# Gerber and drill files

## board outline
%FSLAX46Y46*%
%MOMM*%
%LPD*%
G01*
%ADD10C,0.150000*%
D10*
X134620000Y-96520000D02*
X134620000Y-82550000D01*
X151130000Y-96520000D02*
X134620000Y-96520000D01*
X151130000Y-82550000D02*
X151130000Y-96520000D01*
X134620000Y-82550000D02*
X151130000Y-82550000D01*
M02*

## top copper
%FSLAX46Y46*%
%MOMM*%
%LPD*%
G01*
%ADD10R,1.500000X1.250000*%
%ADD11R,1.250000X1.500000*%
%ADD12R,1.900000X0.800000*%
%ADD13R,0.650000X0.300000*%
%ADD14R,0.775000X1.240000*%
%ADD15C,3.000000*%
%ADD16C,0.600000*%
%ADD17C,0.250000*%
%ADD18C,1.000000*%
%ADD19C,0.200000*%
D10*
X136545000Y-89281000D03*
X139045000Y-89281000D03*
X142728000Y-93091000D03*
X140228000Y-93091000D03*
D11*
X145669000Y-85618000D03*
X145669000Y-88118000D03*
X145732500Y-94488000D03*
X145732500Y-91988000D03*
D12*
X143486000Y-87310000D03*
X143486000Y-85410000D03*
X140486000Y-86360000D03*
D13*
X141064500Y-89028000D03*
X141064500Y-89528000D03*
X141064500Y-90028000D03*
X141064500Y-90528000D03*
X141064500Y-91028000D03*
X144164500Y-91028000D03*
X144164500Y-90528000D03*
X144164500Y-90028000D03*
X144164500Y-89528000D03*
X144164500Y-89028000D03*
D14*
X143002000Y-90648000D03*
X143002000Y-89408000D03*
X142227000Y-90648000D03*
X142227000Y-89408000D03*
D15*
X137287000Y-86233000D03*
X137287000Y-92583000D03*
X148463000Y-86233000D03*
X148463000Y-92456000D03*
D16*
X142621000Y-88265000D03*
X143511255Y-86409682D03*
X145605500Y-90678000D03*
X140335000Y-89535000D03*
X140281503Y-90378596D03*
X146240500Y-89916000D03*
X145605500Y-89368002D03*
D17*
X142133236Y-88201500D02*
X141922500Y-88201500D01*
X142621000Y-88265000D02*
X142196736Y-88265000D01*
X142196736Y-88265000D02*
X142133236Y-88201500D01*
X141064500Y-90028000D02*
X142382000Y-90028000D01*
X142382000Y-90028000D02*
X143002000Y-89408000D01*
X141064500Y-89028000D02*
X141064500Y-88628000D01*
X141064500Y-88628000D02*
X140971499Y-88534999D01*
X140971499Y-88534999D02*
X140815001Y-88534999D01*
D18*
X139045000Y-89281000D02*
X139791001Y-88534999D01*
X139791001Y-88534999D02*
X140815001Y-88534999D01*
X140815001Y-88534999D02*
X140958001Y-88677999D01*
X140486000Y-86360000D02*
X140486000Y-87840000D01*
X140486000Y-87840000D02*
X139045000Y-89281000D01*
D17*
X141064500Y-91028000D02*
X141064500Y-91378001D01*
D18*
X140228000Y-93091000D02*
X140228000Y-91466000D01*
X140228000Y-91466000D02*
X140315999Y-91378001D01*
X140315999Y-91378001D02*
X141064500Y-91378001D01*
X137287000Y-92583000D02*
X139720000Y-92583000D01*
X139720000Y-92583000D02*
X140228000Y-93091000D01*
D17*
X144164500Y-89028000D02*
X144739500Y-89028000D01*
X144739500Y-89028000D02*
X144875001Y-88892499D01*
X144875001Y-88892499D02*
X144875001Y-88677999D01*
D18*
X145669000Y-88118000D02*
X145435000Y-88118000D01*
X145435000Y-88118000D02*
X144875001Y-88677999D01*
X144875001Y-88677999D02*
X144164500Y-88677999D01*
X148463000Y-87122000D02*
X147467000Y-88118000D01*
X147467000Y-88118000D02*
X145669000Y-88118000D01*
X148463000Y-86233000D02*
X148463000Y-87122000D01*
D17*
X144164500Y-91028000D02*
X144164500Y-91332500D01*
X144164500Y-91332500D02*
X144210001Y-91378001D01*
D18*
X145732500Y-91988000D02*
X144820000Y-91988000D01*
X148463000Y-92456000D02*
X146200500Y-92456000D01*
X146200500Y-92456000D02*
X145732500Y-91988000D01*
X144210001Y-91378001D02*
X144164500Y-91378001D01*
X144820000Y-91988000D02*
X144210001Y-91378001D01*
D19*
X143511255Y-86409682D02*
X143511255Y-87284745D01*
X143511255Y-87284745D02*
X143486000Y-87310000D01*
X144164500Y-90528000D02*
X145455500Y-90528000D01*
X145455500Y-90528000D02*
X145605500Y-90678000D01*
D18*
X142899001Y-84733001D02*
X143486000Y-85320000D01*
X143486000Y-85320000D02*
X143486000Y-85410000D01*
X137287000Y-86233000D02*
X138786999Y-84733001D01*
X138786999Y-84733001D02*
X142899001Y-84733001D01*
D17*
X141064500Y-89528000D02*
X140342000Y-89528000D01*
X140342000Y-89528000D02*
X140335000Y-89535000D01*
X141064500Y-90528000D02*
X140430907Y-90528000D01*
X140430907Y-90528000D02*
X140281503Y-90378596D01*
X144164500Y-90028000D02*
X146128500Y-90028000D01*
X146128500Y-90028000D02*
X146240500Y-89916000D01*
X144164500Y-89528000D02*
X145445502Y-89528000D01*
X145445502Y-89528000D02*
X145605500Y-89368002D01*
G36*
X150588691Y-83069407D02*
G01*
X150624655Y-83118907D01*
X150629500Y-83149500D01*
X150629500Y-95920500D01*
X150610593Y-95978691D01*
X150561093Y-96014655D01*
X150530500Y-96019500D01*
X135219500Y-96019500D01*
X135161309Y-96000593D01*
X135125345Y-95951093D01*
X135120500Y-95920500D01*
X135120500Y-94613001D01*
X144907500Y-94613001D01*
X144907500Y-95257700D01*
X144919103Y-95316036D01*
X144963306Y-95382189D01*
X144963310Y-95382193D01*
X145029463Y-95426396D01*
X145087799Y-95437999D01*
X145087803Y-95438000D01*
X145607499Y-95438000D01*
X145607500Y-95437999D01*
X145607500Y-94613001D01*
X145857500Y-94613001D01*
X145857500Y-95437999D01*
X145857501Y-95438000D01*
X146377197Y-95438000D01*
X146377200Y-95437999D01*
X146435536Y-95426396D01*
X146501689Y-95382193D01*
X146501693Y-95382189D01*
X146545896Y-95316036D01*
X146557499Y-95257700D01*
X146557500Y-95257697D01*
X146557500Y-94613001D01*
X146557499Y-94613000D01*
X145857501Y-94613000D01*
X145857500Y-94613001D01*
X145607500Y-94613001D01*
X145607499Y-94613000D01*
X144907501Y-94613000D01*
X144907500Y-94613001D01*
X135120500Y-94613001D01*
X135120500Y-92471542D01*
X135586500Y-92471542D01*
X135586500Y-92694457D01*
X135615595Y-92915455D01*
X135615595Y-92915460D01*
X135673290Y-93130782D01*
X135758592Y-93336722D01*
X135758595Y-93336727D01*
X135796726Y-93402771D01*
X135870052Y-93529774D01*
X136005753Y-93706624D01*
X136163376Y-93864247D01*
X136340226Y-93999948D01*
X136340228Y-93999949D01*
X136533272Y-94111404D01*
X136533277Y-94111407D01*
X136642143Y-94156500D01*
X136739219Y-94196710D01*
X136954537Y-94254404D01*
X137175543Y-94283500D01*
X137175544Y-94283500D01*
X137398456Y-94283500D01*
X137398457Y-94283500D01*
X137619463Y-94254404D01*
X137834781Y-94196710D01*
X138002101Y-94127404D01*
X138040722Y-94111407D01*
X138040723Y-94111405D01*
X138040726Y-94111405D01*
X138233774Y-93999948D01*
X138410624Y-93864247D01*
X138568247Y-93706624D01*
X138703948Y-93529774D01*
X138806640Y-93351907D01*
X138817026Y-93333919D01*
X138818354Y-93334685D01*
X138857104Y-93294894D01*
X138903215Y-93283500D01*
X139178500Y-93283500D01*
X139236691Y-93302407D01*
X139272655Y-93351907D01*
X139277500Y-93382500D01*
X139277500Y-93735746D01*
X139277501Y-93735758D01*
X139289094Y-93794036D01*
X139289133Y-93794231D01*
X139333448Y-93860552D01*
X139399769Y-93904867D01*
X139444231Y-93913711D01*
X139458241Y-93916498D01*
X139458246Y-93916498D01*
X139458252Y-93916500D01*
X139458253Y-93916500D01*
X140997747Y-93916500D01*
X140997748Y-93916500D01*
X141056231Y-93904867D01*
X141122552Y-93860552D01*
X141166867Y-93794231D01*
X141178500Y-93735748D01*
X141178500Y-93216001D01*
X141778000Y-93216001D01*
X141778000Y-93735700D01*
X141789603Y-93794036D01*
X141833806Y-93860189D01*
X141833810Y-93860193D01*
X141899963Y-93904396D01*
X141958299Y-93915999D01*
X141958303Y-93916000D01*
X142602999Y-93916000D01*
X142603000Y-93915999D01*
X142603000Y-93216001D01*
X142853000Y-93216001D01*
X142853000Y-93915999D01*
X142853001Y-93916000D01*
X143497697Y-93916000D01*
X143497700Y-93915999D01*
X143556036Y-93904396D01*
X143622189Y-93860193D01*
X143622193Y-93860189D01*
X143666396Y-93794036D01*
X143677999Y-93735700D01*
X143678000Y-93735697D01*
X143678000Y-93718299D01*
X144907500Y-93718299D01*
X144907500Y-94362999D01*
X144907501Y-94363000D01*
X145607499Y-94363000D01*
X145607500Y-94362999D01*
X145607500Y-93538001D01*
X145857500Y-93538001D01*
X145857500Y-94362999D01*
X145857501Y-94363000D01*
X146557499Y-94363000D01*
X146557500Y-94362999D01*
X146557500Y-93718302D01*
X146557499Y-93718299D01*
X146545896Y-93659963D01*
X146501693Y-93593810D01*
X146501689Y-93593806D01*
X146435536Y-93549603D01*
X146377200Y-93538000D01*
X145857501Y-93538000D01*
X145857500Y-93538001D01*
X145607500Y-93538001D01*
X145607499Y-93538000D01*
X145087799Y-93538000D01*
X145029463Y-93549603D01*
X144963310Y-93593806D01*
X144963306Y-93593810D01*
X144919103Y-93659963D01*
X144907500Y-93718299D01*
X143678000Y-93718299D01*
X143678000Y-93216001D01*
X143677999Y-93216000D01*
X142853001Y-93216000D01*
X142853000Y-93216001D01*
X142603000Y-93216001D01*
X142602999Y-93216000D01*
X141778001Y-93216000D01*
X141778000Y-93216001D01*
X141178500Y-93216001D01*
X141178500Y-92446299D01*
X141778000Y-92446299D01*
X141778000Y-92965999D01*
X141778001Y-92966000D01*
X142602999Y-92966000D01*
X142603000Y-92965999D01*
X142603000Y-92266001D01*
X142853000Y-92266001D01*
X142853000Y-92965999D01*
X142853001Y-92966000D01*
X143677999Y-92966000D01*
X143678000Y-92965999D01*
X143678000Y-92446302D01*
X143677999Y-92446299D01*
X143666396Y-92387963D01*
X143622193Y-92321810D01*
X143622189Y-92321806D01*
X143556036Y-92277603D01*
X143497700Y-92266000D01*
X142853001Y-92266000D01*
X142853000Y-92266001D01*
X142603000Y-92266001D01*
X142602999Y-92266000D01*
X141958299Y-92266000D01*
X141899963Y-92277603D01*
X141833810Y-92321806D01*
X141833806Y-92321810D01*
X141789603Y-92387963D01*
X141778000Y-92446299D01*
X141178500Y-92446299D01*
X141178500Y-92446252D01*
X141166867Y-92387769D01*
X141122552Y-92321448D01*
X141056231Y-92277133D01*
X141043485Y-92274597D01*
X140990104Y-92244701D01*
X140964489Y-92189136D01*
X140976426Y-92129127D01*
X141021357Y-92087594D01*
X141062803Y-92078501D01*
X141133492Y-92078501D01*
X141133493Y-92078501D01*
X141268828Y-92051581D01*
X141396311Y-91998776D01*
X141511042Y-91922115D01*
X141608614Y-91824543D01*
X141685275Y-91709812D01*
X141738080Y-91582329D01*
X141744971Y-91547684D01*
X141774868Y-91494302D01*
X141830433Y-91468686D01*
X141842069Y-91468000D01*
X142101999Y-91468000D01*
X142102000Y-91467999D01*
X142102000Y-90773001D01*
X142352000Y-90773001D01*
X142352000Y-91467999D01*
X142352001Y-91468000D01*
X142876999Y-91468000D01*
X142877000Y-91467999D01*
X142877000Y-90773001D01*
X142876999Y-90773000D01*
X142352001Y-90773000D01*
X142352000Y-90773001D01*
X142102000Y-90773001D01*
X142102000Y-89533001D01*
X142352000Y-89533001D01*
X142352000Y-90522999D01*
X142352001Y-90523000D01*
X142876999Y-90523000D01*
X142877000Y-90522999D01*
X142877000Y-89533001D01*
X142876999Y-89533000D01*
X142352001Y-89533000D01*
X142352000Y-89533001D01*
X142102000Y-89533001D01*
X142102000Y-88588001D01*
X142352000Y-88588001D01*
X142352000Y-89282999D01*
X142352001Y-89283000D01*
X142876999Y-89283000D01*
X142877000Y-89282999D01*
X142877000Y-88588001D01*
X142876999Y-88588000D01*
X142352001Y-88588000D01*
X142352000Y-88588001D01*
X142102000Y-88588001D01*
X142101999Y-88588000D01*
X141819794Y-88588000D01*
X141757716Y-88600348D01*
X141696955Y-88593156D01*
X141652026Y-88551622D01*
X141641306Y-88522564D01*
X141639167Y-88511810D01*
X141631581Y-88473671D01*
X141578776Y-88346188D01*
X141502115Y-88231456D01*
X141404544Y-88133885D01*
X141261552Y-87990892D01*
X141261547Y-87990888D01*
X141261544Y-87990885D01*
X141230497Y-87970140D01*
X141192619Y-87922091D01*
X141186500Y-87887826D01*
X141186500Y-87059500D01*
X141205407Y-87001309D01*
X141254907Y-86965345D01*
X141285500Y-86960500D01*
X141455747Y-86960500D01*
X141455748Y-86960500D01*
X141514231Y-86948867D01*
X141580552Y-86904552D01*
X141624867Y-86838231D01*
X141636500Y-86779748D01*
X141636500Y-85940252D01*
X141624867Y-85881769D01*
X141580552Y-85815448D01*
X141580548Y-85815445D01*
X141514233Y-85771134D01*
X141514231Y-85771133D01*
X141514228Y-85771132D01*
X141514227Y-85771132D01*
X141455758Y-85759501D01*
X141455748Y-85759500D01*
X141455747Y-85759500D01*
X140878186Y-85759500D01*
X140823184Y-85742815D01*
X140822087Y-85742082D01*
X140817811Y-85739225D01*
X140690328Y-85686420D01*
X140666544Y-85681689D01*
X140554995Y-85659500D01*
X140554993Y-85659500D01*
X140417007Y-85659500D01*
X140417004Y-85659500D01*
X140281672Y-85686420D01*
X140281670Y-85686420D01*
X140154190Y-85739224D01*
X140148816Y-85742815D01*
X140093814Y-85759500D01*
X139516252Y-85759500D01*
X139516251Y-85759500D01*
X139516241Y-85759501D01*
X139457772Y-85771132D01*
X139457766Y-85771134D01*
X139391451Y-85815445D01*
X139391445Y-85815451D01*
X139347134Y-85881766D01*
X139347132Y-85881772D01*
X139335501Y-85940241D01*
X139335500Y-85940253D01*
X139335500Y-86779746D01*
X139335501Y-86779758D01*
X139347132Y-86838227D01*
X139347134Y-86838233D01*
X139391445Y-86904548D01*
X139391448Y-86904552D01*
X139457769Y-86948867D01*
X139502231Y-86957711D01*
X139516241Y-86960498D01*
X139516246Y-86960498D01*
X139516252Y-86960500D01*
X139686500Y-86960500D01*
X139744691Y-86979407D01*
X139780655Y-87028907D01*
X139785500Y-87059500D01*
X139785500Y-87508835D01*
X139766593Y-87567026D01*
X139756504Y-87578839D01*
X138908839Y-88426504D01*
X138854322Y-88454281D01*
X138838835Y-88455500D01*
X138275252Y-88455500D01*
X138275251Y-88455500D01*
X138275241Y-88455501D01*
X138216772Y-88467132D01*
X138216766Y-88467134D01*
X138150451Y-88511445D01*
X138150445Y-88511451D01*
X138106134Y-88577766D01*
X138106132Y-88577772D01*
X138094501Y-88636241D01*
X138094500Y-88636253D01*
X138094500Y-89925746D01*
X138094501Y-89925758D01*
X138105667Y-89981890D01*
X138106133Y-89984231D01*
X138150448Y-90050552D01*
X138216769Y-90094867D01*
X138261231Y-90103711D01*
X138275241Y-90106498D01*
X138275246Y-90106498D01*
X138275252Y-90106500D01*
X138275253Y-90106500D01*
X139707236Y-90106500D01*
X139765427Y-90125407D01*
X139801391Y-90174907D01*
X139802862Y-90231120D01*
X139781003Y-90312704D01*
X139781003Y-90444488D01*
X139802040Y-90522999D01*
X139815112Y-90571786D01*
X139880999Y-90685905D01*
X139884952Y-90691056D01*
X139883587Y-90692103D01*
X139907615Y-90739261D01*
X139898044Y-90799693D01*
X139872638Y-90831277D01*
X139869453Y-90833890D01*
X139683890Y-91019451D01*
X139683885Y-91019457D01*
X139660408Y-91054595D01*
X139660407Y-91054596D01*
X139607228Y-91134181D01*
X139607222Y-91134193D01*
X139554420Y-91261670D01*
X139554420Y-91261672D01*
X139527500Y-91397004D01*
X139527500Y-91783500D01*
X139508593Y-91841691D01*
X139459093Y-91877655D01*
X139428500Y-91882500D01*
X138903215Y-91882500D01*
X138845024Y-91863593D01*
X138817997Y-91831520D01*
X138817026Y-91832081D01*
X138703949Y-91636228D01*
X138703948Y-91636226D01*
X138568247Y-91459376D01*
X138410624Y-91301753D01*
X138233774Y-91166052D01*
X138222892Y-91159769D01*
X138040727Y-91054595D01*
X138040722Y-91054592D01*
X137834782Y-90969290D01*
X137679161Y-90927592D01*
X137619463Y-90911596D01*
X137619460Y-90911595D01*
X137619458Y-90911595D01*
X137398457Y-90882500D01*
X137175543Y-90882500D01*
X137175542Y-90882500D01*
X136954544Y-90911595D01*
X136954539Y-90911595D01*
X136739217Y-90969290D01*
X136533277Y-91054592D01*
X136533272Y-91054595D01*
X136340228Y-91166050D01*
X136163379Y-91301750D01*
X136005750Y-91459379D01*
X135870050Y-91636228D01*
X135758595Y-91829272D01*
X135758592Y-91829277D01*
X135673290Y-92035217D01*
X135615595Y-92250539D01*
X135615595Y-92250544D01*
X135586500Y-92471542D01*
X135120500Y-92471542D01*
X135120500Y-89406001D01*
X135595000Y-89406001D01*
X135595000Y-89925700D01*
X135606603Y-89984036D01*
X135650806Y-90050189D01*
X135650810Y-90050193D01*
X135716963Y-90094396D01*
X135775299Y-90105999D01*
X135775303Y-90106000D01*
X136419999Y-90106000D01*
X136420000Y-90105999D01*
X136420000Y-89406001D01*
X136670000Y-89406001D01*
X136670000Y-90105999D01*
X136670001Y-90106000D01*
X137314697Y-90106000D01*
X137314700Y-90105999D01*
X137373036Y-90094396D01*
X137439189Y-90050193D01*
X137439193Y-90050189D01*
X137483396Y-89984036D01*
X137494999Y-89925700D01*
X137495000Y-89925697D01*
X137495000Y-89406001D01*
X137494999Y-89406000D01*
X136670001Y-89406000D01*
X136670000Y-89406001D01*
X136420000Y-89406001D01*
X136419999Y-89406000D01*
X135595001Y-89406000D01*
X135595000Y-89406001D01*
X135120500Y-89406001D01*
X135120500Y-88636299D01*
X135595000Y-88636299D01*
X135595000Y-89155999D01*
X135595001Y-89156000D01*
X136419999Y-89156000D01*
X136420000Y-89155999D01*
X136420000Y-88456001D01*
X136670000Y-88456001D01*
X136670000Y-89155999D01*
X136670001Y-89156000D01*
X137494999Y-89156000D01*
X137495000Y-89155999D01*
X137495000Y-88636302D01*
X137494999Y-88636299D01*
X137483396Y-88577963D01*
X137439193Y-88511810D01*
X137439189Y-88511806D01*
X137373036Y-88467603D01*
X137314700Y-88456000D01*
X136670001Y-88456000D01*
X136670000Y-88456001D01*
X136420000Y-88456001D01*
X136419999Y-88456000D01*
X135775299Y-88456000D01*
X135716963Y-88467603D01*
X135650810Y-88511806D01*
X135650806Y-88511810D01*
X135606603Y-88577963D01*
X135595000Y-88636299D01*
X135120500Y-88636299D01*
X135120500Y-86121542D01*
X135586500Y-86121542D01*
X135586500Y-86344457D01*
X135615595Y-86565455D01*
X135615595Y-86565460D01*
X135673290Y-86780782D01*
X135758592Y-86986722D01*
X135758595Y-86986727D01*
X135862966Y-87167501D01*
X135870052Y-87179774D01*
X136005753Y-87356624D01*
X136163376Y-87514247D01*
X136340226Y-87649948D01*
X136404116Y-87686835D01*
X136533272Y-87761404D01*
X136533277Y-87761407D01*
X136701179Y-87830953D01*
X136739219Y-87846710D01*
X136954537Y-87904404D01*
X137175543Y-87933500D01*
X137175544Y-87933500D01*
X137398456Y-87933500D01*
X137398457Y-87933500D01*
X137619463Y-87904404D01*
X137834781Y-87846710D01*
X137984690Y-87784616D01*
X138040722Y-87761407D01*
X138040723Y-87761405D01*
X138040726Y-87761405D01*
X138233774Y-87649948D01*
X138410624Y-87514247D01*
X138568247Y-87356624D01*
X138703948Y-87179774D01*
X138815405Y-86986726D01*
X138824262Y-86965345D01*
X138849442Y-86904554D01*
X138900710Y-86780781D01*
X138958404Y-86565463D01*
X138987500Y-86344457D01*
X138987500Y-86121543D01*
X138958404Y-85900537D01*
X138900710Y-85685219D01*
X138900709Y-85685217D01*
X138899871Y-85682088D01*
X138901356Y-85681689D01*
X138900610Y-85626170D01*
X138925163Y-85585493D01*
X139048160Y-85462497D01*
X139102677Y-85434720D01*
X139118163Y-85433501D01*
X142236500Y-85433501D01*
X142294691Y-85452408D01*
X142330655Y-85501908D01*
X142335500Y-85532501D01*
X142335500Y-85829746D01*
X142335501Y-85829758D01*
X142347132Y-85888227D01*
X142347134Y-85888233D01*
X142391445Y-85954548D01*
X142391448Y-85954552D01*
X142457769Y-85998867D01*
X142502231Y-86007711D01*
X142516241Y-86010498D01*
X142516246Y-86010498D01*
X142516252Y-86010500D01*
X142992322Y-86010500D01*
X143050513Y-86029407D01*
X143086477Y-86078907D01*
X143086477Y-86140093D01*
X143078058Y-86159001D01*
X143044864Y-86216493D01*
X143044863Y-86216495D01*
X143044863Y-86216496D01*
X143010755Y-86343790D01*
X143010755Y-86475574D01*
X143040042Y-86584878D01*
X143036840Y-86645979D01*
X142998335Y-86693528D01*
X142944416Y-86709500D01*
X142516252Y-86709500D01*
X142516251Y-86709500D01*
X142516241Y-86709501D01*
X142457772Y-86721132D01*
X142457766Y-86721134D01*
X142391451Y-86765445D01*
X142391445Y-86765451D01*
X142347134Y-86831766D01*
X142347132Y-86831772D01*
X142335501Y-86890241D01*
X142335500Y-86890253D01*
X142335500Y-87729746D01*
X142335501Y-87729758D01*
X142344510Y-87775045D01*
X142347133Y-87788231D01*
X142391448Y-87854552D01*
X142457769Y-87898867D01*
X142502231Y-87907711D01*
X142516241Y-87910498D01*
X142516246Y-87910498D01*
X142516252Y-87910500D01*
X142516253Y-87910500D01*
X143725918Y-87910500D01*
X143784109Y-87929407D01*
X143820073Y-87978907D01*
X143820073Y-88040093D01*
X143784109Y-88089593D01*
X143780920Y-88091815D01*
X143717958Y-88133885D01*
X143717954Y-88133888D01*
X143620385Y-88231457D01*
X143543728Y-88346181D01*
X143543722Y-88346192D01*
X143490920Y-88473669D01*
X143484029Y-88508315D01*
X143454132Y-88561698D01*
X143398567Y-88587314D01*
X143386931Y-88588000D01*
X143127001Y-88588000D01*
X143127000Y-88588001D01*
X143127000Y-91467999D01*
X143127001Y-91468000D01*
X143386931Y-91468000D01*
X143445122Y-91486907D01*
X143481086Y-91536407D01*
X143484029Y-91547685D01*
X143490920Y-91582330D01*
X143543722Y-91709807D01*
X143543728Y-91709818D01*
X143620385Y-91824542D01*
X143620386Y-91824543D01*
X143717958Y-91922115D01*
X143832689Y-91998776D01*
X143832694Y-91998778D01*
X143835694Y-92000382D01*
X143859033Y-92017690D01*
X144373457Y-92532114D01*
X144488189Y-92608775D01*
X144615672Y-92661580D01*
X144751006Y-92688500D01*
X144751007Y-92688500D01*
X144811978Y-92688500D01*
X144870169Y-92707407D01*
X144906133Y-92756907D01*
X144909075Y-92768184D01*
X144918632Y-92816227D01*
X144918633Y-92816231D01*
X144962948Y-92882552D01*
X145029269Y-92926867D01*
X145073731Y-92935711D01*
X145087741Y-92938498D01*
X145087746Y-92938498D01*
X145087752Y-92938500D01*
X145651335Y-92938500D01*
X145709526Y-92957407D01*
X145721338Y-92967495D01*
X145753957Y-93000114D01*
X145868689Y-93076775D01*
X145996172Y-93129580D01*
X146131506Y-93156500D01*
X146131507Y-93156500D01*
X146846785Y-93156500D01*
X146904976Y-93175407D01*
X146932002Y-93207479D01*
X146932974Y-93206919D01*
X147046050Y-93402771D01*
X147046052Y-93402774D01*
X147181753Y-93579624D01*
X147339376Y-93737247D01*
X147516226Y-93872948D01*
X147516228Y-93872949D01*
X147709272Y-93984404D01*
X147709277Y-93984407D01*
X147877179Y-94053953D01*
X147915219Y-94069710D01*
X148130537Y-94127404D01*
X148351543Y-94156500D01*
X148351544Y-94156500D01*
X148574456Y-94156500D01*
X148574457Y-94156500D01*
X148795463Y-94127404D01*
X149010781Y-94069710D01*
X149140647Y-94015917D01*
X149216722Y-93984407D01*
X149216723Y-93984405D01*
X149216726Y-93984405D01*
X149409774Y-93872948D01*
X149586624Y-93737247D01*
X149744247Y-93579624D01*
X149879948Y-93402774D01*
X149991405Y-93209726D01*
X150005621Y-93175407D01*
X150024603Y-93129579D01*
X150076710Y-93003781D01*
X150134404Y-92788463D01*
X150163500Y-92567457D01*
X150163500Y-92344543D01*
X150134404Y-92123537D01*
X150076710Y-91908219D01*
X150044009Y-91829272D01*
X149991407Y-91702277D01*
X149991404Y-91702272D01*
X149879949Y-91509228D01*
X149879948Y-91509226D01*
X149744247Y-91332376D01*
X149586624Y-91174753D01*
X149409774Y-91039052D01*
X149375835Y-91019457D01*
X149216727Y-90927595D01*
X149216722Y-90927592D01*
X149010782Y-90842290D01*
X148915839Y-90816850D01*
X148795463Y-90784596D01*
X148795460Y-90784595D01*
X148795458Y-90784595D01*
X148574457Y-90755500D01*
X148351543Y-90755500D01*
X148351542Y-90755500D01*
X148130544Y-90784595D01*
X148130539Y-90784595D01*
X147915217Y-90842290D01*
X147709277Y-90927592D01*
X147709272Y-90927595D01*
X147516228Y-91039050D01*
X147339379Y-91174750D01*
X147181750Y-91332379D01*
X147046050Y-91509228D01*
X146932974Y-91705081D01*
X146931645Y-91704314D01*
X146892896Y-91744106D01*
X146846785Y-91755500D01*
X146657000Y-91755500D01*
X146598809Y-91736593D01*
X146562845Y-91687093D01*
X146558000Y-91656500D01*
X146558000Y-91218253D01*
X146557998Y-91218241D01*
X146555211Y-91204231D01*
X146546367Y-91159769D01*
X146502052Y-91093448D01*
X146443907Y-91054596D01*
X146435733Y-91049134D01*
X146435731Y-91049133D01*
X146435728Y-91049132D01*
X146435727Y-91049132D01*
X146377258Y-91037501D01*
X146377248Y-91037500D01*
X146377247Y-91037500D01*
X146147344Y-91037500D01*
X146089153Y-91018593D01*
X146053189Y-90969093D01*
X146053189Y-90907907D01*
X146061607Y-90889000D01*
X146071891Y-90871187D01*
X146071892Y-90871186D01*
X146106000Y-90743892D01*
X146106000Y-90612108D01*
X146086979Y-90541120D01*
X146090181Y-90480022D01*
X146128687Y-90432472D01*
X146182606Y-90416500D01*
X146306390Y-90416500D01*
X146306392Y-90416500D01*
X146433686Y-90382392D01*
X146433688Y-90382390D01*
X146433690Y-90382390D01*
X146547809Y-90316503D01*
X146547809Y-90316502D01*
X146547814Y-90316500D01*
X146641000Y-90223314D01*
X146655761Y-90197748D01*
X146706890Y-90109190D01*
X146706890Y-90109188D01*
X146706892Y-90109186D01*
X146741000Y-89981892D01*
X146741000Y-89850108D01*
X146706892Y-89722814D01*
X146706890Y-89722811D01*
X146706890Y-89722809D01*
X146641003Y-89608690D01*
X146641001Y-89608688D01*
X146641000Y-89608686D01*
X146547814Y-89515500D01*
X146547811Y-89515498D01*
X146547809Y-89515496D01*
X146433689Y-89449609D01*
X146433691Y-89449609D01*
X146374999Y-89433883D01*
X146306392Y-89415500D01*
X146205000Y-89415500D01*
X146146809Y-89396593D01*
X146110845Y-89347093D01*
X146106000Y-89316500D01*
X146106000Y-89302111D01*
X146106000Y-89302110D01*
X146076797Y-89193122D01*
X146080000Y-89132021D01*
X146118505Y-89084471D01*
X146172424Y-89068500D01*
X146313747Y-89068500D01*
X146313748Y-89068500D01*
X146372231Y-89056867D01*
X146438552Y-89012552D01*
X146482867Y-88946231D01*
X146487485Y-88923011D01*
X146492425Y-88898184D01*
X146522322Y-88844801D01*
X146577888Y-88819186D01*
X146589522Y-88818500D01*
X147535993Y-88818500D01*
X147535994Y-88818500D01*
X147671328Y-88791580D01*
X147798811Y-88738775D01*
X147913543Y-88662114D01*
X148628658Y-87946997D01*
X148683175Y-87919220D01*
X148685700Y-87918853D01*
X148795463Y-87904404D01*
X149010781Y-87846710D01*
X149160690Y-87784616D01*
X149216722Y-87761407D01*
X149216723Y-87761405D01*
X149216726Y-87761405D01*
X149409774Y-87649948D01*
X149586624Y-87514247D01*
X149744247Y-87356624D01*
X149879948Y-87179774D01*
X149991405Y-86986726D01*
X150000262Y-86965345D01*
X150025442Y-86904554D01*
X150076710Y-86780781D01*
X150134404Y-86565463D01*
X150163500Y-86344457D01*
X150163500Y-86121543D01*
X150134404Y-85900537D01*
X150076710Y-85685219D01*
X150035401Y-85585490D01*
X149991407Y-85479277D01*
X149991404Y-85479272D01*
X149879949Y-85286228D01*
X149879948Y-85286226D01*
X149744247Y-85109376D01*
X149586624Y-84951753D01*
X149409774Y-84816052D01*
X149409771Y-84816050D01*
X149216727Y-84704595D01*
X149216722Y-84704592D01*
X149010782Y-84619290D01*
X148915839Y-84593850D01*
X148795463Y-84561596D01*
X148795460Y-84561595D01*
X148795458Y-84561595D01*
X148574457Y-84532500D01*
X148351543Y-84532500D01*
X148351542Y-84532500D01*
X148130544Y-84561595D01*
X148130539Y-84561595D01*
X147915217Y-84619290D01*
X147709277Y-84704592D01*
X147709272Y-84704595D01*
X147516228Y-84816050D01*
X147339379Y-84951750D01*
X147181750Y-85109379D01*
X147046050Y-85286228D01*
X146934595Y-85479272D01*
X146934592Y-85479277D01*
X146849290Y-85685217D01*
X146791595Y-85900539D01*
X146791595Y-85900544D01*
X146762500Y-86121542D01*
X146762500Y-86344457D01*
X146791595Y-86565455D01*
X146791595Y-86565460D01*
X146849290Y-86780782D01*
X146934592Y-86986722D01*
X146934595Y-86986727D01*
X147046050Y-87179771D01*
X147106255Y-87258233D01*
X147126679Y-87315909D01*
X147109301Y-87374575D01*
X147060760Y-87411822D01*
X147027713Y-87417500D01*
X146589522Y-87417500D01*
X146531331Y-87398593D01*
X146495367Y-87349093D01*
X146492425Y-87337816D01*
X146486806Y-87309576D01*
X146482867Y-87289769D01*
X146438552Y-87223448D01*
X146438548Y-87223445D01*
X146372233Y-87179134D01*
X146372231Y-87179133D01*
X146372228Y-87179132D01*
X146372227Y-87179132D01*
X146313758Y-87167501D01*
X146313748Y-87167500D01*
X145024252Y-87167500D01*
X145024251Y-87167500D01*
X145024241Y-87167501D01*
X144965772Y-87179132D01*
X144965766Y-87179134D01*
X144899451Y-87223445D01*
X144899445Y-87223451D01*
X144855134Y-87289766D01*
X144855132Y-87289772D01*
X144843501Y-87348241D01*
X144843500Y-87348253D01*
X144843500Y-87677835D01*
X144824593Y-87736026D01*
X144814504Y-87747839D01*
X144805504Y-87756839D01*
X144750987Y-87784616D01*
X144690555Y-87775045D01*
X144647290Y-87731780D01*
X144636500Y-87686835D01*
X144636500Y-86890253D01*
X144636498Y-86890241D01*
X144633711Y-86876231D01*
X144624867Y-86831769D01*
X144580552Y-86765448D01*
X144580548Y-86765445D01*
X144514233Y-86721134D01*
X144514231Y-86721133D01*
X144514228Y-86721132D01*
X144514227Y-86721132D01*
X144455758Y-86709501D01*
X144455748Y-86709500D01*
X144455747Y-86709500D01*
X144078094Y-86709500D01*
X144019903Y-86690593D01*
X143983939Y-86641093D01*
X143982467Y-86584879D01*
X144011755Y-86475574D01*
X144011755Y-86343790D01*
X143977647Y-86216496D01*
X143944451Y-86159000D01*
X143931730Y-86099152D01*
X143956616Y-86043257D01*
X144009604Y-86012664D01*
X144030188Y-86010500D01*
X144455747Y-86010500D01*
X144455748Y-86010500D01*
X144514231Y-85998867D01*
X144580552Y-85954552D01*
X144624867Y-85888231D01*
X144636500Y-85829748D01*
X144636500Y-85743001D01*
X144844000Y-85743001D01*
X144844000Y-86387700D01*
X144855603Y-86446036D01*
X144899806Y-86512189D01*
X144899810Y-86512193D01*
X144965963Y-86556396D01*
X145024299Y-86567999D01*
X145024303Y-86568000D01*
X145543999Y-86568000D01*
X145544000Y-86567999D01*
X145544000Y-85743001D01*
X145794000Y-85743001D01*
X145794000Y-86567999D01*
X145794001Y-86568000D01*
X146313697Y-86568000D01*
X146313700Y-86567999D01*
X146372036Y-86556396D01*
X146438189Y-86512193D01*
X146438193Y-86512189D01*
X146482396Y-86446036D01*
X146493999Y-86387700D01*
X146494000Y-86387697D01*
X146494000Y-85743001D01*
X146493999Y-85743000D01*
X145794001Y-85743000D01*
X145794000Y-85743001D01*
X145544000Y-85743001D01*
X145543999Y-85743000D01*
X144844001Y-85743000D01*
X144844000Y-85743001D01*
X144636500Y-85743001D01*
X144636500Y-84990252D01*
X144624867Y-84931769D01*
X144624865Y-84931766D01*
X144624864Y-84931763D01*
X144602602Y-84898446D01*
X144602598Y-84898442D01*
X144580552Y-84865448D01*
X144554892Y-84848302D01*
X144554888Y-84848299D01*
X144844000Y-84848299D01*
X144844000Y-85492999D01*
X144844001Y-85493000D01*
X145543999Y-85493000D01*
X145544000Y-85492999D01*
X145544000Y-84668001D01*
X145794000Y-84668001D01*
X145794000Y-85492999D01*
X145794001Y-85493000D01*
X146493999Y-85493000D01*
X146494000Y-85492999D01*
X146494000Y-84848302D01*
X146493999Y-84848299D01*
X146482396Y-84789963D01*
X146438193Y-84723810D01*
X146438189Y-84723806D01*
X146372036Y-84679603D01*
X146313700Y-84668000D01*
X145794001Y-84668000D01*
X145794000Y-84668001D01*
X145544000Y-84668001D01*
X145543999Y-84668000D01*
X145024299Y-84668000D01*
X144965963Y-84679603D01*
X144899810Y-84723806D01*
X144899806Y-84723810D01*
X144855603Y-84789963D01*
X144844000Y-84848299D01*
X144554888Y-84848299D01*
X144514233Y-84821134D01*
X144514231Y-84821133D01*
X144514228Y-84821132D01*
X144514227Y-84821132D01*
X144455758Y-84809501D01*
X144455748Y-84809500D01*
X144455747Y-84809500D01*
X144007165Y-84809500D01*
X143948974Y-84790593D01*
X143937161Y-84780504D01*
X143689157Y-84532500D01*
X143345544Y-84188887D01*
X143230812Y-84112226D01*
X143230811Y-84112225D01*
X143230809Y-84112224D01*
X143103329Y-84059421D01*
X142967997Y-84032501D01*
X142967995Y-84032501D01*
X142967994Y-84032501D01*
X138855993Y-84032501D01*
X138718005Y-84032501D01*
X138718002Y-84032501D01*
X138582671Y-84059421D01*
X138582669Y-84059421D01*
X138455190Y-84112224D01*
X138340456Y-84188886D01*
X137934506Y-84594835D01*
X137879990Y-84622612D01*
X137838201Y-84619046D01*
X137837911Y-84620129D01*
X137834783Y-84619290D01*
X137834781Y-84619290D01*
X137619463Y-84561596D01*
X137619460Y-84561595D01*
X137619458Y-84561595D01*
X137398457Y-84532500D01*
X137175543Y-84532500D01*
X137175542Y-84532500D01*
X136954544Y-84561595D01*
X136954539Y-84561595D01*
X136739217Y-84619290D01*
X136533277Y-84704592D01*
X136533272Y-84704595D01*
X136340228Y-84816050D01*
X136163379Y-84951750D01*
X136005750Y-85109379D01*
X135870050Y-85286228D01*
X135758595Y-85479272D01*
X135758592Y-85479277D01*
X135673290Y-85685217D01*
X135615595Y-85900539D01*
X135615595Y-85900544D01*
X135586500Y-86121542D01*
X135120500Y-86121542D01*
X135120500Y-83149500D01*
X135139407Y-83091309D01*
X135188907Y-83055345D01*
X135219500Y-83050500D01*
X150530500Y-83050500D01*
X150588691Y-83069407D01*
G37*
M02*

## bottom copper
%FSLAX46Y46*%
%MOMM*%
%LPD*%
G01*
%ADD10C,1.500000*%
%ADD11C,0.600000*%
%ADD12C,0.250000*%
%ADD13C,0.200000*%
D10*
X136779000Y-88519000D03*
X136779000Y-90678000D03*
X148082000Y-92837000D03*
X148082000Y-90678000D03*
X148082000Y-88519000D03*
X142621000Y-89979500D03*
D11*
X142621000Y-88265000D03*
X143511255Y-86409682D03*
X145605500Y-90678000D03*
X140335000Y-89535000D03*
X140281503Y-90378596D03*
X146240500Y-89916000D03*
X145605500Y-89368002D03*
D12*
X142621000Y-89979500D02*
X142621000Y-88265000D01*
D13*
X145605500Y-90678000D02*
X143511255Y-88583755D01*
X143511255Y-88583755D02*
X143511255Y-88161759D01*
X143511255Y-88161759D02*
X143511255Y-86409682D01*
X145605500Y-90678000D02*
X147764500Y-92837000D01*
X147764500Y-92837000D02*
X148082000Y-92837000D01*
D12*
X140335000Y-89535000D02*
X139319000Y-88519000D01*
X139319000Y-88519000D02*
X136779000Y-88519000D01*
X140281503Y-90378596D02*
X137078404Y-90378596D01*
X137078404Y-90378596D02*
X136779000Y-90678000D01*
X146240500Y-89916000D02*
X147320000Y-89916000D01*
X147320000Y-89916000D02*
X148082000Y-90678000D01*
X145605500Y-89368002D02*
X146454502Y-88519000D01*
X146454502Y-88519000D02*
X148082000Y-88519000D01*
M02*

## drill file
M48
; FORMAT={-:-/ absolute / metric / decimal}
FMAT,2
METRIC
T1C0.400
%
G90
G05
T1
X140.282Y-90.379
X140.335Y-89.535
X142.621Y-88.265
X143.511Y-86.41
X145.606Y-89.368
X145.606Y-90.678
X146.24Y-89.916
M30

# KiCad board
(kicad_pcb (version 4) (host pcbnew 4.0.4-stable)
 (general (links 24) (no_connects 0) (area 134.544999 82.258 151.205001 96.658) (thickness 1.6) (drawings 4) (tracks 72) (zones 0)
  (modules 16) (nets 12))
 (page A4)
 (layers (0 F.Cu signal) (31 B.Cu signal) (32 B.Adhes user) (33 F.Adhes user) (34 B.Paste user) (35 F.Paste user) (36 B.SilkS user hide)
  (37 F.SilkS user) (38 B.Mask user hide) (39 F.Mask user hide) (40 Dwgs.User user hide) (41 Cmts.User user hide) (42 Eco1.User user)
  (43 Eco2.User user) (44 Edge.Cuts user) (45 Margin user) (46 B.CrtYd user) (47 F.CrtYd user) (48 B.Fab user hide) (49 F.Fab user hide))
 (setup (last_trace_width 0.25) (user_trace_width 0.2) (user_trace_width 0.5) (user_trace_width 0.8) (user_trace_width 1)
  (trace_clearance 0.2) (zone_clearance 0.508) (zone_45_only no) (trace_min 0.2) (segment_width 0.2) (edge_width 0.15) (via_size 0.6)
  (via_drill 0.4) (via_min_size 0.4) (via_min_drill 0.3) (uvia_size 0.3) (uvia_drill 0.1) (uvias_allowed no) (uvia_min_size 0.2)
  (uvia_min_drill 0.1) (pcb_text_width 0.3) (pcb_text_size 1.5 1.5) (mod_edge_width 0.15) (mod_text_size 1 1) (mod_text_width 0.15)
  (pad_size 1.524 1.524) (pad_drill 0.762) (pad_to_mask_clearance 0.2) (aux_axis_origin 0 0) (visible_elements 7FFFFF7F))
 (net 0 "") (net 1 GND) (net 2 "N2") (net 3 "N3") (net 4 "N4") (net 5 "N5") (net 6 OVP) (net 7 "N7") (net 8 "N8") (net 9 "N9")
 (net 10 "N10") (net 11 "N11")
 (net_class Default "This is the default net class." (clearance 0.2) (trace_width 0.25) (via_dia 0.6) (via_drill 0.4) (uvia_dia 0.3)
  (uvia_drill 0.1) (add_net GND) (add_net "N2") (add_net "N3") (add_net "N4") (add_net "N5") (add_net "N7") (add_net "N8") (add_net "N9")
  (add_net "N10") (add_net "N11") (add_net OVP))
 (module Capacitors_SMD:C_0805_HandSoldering (layer F.Cu) (at 137.795 89.281)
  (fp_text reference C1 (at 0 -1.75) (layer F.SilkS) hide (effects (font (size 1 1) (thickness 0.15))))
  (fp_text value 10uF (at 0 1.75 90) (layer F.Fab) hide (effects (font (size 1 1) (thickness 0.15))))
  (pad 1 smd rect (at -1.25 0) (size 1.5 1.25) (layers F.Cu F.Paste F.Mask) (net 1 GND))
  (pad 2 smd rect (at 1.25 0) (size 1.5 1.25) (layers F.Cu F.Paste F.Mask) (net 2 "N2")))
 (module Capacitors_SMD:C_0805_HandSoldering (layer F.Cu) (at 141.478 93.091 180)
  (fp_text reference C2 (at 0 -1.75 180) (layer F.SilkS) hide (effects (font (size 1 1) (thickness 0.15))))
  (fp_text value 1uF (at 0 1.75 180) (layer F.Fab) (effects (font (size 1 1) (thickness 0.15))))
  (pad 1 smd rect (at -1.25 0 180) (size 1.5 1.25) (layers F.Cu F.Paste F.Mask) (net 1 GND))
  (pad 2 smd rect (at 1.25 0 180) (size 1.5 1.25) (layers F.Cu F.Paste F.Mask) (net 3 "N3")))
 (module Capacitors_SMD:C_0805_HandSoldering (layer F.Cu) (at 145.669 86.868 270)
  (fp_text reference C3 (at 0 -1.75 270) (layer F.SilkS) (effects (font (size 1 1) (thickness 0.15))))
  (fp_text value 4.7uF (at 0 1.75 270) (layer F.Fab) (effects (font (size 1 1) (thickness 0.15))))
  (pad 1 smd rect (at -1.25 0 270) (size 1.5 1.25) (layers F.Cu F.Paste F.Mask) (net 1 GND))
  (pad 2 smd rect (at 1.25 0 270) (size 1.5 1.25) (layers F.Cu F.Paste F.Mask) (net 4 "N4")))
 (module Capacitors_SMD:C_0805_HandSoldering (layer F.Cu) (at 145.7325 93.238 90)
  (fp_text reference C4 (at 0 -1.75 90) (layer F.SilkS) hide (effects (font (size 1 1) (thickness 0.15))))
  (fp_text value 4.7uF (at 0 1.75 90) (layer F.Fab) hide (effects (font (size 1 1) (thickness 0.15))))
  (pad 1 smd rect (at -1.25 0 90) (size 1.5 1.25) (layers F.Cu F.Paste F.Mask) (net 1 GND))
  (pad 2 smd rect (at 1.25 0 90) (size 1.5 1.25) (layers F.Cu F.Paste F.Mask) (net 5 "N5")))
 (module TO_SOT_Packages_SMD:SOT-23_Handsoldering (layer F.Cu) (at 141.986 86.36 180)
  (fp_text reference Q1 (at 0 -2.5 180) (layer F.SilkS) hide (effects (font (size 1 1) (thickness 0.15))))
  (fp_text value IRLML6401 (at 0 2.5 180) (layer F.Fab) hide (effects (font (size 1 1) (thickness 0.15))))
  (pad 1 smd rect (at -1.5 -0.95 180) (size 1.9 0.8) (layers F.Cu F.Paste F.Mask) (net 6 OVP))
  (pad 2 smd rect (at -1.5 0.95 180) (size 1.9 0.8) (layers F.Cu F.Paste F.Mask) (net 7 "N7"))
  (pad 3 smd rect (at 1.5 0 180) (size 1.9 0.8) (layers F.Cu F.Paste F.Mask) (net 2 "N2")))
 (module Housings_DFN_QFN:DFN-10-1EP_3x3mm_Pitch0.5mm (layer F.Cu) (at 142.6145 90.028)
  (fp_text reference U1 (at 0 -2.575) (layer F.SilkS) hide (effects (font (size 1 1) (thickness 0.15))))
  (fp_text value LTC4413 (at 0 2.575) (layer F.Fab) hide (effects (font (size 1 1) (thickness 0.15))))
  (pad 1 smd rect (at -1.55 -1) (size 0.65 0.3) (layers F.Cu F.Paste F.Mask) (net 2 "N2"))
  (pad 2 smd rect (at -1.55 -0.5) (size 0.65 0.3) (layers F.Cu F.Paste F.Mask) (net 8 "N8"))
  (pad 3 smd rect (at -1.55 0) (size 0.65 0.3) (layers F.Cu F.Paste F.Mask) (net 1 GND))
  (pad 4 smd rect (at -1.55 0.5) (size 0.65 0.3) (layers F.Cu F.Paste F.Mask) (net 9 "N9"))
  (pad 5 smd rect (at -1.55 1) (size 0.65 0.3) (layers F.Cu F.Paste F.Mask) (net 3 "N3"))
  (pad 6 smd rect (at 1.55 1) (size 0.65 0.3) (layers F.Cu F.Paste F.Mask) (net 5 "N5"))
  (pad 7 smd rect (at 1.55 0.5) (size 0.65 0.3) (layers F.Cu F.Paste F.Mask) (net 6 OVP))
  (pad 8 smd rect (at 1.55 0) (size 0.65 0.3) (layers F.Cu F.Paste F.Mask) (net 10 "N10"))
  (pad 9 smd rect (at 1.55 -0.5) (size 0.65 0.3) (layers F.Cu F.Paste F.Mask) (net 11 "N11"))
  (pad 10 smd rect (at 1.55 -1) (size 0.65 0.3) (layers F.Cu F.Paste F.Mask) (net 4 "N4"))
  (pad 11 smd rect (at 0.3875 0.62) (size 0.775 1.24) (layers F.Cu F.Paste F.Mask) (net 1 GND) (solder_paste_margin_ratio -0.2))
  (pad 11 smd rect (at 0.3875 -0.62) (size 0.775 1.24) (layers F.Cu F.Paste F.Mask) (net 1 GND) (solder_paste_margin_ratio -0.2))
  (pad 11 smd rect (at -0.3875 0.62) (size 0.775 1.24) (layers F.Cu F.Paste F.Mask) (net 1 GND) (solder_paste_margin_ratio -0.2))
  (pad 11 smd rect (at -0.3875 -0.62) (size 0.775 1.24) (layers F.Cu F.Paste F.Mask) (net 1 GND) (solder_paste_margin_ratio -0.2)))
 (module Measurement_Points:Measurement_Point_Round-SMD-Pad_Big (layer F.Cu) (at 137.287 86.233)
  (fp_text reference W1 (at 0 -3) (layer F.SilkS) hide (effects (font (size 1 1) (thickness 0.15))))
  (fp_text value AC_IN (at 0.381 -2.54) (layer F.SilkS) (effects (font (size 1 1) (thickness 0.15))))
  (pad 1 smd circle (at 0 0) (size 3 3) (layers F.Cu F.Mask) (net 7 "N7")))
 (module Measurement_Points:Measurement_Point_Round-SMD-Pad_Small (layer B.Cu) (at 136.779 88.519)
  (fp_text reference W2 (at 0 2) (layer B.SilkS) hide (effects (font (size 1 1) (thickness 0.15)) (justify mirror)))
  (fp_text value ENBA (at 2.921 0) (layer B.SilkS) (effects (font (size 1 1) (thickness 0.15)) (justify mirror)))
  (pad 1 smd circle (at 0 0) (size 1.5 1.5) (layers B.Cu B.Mask) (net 8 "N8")))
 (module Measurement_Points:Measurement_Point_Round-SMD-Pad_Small (layer B.Cu) (at 136.779 90.678)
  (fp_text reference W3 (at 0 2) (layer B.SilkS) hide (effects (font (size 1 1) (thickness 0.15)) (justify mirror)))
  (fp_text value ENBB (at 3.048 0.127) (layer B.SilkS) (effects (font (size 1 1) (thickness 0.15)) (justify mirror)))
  (pad 1 smd circle (at 0 0) (size 1.5 1.5) (layers B.Cu B.Mask) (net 9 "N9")))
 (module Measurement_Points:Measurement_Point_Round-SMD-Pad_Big (layer F.Cu) (at 137.287 92.583)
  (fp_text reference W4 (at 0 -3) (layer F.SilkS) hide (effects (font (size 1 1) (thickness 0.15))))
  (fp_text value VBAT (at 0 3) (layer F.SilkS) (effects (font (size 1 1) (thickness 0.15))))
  (pad 1 smd circle (at 0 0) (size 3 3) (layers F.Cu F.Mask) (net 3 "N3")))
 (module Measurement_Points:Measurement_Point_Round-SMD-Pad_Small (layer B.Cu) (at 148.082 92.837)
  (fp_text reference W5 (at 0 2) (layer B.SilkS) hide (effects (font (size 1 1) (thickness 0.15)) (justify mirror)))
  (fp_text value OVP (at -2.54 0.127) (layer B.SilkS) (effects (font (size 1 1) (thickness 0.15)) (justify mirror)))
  (pad 1 smd circle (at 0 0) (size 1.5 1.5) (layers B.Cu B.Mask) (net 6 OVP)))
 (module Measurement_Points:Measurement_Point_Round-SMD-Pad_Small (layer B.Cu) (at 148.082 90.678)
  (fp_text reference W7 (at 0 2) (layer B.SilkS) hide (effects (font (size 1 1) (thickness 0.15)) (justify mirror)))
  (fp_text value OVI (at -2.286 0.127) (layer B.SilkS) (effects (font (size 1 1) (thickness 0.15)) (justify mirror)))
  (pad 1 smd circle (at 0 0) (size 1.5 1.5) (layers B.Cu B.Mask) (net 10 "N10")))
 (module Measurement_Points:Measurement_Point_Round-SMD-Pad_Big (layer F.Cu) (at 148.463 86.233)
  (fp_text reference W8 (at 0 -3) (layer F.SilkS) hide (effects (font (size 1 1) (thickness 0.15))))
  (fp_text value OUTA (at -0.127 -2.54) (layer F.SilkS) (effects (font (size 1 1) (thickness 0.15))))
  (pad 1 smd circle (at 0 0) (size 3 3) (layers F.Cu F.Mask) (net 4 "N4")))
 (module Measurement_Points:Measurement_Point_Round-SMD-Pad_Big (layer F.Cu) (at 148.463 92.456)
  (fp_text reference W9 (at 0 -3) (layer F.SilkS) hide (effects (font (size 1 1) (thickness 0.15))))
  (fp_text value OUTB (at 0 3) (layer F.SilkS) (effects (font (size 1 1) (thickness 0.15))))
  (pad 1 smd circle (at 0 0) (size 3 3) (layers F.Cu F.Mask) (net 5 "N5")))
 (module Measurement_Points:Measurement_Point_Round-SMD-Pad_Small (layer B.Cu) (at 148.082 88.519)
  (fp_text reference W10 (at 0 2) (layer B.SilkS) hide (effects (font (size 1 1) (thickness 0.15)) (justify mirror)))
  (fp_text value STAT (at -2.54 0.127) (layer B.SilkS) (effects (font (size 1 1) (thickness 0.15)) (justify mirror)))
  (pad 1 smd circle (at 0 0) (size 1.5 1.5) (layers B.Cu B.Mask) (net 11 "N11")))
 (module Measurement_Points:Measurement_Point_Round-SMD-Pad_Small (layer B.Cu) (at 142.621 89.9795)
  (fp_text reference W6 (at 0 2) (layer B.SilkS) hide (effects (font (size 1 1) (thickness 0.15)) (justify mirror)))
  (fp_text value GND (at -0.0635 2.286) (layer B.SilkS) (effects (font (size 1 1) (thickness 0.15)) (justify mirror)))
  (pad 1 smd circle (at 0 0) (size 1.5 1.5) (layers B.Cu B.Mask) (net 1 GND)))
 (gr_line (start 134.62 96.52) (end 134.62 82.55) (layer Edge.Cuts) (width 0.15))
 (gr_line (start 151.13 96.52) (end 134.62 96.52) (layer Edge.Cuts) (width 0.15))
 (gr_line (start 151.13 82.55) (end 151.13 96.52) (layer Edge.Cuts) (width 0.15))
 (gr_line (start 134.62 82.55) (end 151.13 82.55) (layer Edge.Cuts) (width 0.15))
 (segment (start 142.133236 88.2015) (end 141.9225 88.2015) (width 0.25) (layer F.Cu) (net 1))
 (segment (start 142.621 88.265) (end 142.196736 88.265) (width 0.25) (layer F.Cu) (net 1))
 (segment (start 142.196736 88.265) (end 142.133236 88.2015) (width 0.25) (layer F.Cu) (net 1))
 (segment (start 142.621 89.9795) (end 142.621 88.265) (width 0.25) (layer B.Cu) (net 1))
 (via (at 142.621 88.265) (size 0.6) (drill 0.4) (layers F.Cu B.Cu) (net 1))
 (segment (start 141.0645 90.028) (end 142.382 90.028) (width 0.25) (layer F.Cu) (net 1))
 (segment (start 142.382 90.028) (end 143.002 89.408) (width 0.25) (layer F.Cu) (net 1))
 (segment (start 141.0645 89.028) (end 141.0645 88.628) (width 0.25) (layer F.Cu) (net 2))
 (segment (start 141.0645 88.628) (end 140.971499 88.534999) (width 0.25) (layer F.Cu) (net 2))
 (segment (start 140.971499 88.534999) (end 140.815001 88.534999) (width 0.25) (layer F.Cu) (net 2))
 (segment (start 139.045 89.281) (end 139.791001 88.534999) (width 1) (layer F.Cu) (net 2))
 (segment (start 139.791001 88.534999) (end 140.815001 88.534999) (width 1) (layer F.Cu) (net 2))
 (segment (start 140.815001 88.534999) (end 140.958001 88.677999) (width 1) (layer F.Cu) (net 2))
 (segment (start 140.486 86.36) (end 140.486 87.84) (width 1) (layer F.Cu) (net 2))
 (segment (start 140.486 87.84) (end 139.045 89.281) (width 1) (layer F.Cu) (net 2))
 (segment (start 141.0645 91.028) (end 141.0645 91.378001) (width 0.25) (layer F.Cu) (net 3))
 (segment (start 140.228 93.091) (end 140.228 91.466) (width 1) (layer F.Cu) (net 3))
 (segment (start 140.228 91.466) (end 140.315999 91.378001) (width 1) (layer F.Cu) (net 3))
 (segment (start 140.315999 91.378001) (end 141.0645 91.378001) (width 1) (layer F.Cu) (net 3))
 (segment (start 137.287 92.583) (end 139.72 92.583) (width 1) (layer F.Cu) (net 3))
 (segment (start 139.72 92.583) (end 140.228 93.091) (width 1) (layer F.Cu) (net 3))
 (segment (start 144.1645 89.028) (end 144.7395 89.028) (width 0.25) (layer F.Cu) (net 4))
 (segment (start 144.7395 89.028) (end 144.875001 88.892499) (width 0.25) (layer F.Cu) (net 4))
 (segment (start 144.875001 88.892499) (end 144.875001 88.677999) (width 0.25) (layer F.Cu) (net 4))
 (segment (start 145.669 88.118) (end 145.435 88.118) (width 1) (layer F.Cu) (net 4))
 (segment (start 145.435 88.118) (end 144.875001 88.677999) (width 1) (layer F.Cu) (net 4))
 (segment (start 144.875001 88.677999) (end 144.1645 88.677999) (width 1) (layer F.Cu) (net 4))
 (segment (start 148.463 87.122) (end 147.467 88.118) (width 1) (layer F.Cu) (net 4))
 (segment (start 147.467 88.118) (end 145.669 88.118) (width 1) (layer F.Cu) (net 4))
 (segment (start 148.463 86.233) (end 148.463 87.122) (width 1) (layer F.Cu) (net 4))
 (segment (start 144.1645 91.028) (end 144.1645 91.3325) (width 0.25) (layer F.Cu) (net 5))
 (segment (start 144.1645 91.3325) (end 144.210001 91.378001) (width 0.25) (layer F.Cu) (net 5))
 (segment (start 145.7325 91.988) (end 144.82 91.988) (width 1) (layer F.Cu) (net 5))
 (segment (start 148.463 92.456) (end 146.2005 92.456) (width 1) (layer F.Cu) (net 5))
 (segment (start 146.2005 92.456) (end 145.7325 91.988) (width 1) (layer F.Cu) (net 5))
 (segment (start 144.210001 91.378001) (end 144.1645 91.378001) (width 1) (layer F.Cu) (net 5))
 (segment (start 144.82 91.988) (end 144.210001 91.378001) (width 1) (layer F.Cu) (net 5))
 (segment (start 143.511255 86.409682) (end 143.511255 87.284745) (width 0.2) (layer F.Cu) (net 6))
 (segment (start 143.511255 87.284745) (end 143.486 87.31) (width 0.2) (layer F.Cu) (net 6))
 (segment (start 145.6055 90.678) (end 143.511255 88.583755) (width 0.2) (layer B.Cu) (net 6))
 (segment (start 143.511255 88.583755) (end 143.511255 88.161759) (width 0.2) (layer B.Cu) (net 6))
 (segment (start 143.511255 88.161759) (end 143.511255 86.409682) (width 0.2) (layer B.Cu) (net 6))
 (via (at 143.511255 86.409682) (size 0.6) (drill 0.4) (layers F.Cu B.Cu) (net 6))
 (segment (start 145.6055 90.678) (end 147.7645 92.837) (width 0.2) (layer B.Cu) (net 6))
 (segment (start 147.7645 92.837) (end 148.082 92.837) (width 0.2) (layer B.Cu) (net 6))
 (segment (start 144.1645 90.528) (end 145.4555 90.528) (width 0.2) (layer F.Cu) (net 6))
 (segment (start 145.4555 90.528) (end 145.6055 90.678) (width 0.2) (layer F.Cu) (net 6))
 (via (at 145.6055 90.678) (size 0.6) (drill 0.4) (layers F.Cu B.Cu) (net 6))
 (segment (start 142.899001 84.733001) (end 143.486 85.32) (width 1) (layer F.Cu) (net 7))
 (segment (start 143.486 85.32) (end 143.486 85.41) (width 1) (layer F.Cu) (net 7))
 (segment (start 137.287 86.233) (end 138.786999 84.733001) (width 1) (layer F.Cu) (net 7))
 (segment (start 138.786999 84.733001) (end 142.899001 84.733001) (width 1) (layer F.Cu) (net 7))
 (segment (start 140.335 89.535) (end 139.319 88.519) (width 0.25) (layer B.Cu) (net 8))
 (segment (start 139.319 88.519) (end 136.779 88.519) (width 0.25) (layer B.Cu) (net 8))
 (segment (start 141.0645 89.528) (end 140.342 89.528) (width 0.25) (layer F.Cu) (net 8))
 (segment (start 140.342 89.528) (end 140.335 89.535) (width 0.25) (layer F.Cu) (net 8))
 (via (at 140.335 89.535) (size 0.6) (drill 0.4) (layers F.Cu B.Cu) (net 8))
 (segment (start 140.281503 90.378596) (end 137.078404 90.378596) (width 0.25) (layer B.Cu) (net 9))
 (segment (start 137.078404 90.378596) (end 136.779 90.678) (width 0.25) (layer B.Cu) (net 9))
 (segment (start 141.0645 90.528) (end 140.430907 90.528) (width 0.25) (layer F.Cu) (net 9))
 (segment (start 140.430907 90.528) (end 140.281503 90.378596) (width 0.25) (layer F.Cu) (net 9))
 (via (at 140.281503 90.378596) (size 0.6) (drill 0.4) (layers F.Cu B.Cu) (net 9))
 (segment (start 146.2405 89.916) (end 147.32 89.916) (width 0.25) (layer B.Cu) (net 10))
 (segment (start 147.32 89.916) (end 148.082 90.678) (width 0.25) (layer B.Cu) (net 10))
 (segment (start 144.1645 90.028) (end 146.1285 90.028) (width 0.25) (layer F.Cu) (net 10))
 (segment (start 146.1285 90.028) (end 146.2405 89.916) (width 0.25) (layer F.Cu) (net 10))
 (via (at 146.2405 89.916) (size 0.6) (drill 0.4) (layers F.Cu B.Cu) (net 10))
 (segment (start 145.6055 89.368002) (end 146.454502 88.519) (width 0.25) (layer B.Cu) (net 11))
 (segment (start 146.454502 88.519) (end 148.082 88.519) (width 0.25) (layer B.Cu) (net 11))
 (segment (start 144.1645 89.528) (end 145.445502 89.528) (width 0.25) (layer F.Cu) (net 11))
 (segment (start 145.445502 89.528) (end 145.6055 89.368002) (width 0.25) (layer F.Cu) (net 11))
 (via (at 145.6055 89.368002) (size 0.6) (drill 0.4) (layers F.Cu B.Cu) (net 11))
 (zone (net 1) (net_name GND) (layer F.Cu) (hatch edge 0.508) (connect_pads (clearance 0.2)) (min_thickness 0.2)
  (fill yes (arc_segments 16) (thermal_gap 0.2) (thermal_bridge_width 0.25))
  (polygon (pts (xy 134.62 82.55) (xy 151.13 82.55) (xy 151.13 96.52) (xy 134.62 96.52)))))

